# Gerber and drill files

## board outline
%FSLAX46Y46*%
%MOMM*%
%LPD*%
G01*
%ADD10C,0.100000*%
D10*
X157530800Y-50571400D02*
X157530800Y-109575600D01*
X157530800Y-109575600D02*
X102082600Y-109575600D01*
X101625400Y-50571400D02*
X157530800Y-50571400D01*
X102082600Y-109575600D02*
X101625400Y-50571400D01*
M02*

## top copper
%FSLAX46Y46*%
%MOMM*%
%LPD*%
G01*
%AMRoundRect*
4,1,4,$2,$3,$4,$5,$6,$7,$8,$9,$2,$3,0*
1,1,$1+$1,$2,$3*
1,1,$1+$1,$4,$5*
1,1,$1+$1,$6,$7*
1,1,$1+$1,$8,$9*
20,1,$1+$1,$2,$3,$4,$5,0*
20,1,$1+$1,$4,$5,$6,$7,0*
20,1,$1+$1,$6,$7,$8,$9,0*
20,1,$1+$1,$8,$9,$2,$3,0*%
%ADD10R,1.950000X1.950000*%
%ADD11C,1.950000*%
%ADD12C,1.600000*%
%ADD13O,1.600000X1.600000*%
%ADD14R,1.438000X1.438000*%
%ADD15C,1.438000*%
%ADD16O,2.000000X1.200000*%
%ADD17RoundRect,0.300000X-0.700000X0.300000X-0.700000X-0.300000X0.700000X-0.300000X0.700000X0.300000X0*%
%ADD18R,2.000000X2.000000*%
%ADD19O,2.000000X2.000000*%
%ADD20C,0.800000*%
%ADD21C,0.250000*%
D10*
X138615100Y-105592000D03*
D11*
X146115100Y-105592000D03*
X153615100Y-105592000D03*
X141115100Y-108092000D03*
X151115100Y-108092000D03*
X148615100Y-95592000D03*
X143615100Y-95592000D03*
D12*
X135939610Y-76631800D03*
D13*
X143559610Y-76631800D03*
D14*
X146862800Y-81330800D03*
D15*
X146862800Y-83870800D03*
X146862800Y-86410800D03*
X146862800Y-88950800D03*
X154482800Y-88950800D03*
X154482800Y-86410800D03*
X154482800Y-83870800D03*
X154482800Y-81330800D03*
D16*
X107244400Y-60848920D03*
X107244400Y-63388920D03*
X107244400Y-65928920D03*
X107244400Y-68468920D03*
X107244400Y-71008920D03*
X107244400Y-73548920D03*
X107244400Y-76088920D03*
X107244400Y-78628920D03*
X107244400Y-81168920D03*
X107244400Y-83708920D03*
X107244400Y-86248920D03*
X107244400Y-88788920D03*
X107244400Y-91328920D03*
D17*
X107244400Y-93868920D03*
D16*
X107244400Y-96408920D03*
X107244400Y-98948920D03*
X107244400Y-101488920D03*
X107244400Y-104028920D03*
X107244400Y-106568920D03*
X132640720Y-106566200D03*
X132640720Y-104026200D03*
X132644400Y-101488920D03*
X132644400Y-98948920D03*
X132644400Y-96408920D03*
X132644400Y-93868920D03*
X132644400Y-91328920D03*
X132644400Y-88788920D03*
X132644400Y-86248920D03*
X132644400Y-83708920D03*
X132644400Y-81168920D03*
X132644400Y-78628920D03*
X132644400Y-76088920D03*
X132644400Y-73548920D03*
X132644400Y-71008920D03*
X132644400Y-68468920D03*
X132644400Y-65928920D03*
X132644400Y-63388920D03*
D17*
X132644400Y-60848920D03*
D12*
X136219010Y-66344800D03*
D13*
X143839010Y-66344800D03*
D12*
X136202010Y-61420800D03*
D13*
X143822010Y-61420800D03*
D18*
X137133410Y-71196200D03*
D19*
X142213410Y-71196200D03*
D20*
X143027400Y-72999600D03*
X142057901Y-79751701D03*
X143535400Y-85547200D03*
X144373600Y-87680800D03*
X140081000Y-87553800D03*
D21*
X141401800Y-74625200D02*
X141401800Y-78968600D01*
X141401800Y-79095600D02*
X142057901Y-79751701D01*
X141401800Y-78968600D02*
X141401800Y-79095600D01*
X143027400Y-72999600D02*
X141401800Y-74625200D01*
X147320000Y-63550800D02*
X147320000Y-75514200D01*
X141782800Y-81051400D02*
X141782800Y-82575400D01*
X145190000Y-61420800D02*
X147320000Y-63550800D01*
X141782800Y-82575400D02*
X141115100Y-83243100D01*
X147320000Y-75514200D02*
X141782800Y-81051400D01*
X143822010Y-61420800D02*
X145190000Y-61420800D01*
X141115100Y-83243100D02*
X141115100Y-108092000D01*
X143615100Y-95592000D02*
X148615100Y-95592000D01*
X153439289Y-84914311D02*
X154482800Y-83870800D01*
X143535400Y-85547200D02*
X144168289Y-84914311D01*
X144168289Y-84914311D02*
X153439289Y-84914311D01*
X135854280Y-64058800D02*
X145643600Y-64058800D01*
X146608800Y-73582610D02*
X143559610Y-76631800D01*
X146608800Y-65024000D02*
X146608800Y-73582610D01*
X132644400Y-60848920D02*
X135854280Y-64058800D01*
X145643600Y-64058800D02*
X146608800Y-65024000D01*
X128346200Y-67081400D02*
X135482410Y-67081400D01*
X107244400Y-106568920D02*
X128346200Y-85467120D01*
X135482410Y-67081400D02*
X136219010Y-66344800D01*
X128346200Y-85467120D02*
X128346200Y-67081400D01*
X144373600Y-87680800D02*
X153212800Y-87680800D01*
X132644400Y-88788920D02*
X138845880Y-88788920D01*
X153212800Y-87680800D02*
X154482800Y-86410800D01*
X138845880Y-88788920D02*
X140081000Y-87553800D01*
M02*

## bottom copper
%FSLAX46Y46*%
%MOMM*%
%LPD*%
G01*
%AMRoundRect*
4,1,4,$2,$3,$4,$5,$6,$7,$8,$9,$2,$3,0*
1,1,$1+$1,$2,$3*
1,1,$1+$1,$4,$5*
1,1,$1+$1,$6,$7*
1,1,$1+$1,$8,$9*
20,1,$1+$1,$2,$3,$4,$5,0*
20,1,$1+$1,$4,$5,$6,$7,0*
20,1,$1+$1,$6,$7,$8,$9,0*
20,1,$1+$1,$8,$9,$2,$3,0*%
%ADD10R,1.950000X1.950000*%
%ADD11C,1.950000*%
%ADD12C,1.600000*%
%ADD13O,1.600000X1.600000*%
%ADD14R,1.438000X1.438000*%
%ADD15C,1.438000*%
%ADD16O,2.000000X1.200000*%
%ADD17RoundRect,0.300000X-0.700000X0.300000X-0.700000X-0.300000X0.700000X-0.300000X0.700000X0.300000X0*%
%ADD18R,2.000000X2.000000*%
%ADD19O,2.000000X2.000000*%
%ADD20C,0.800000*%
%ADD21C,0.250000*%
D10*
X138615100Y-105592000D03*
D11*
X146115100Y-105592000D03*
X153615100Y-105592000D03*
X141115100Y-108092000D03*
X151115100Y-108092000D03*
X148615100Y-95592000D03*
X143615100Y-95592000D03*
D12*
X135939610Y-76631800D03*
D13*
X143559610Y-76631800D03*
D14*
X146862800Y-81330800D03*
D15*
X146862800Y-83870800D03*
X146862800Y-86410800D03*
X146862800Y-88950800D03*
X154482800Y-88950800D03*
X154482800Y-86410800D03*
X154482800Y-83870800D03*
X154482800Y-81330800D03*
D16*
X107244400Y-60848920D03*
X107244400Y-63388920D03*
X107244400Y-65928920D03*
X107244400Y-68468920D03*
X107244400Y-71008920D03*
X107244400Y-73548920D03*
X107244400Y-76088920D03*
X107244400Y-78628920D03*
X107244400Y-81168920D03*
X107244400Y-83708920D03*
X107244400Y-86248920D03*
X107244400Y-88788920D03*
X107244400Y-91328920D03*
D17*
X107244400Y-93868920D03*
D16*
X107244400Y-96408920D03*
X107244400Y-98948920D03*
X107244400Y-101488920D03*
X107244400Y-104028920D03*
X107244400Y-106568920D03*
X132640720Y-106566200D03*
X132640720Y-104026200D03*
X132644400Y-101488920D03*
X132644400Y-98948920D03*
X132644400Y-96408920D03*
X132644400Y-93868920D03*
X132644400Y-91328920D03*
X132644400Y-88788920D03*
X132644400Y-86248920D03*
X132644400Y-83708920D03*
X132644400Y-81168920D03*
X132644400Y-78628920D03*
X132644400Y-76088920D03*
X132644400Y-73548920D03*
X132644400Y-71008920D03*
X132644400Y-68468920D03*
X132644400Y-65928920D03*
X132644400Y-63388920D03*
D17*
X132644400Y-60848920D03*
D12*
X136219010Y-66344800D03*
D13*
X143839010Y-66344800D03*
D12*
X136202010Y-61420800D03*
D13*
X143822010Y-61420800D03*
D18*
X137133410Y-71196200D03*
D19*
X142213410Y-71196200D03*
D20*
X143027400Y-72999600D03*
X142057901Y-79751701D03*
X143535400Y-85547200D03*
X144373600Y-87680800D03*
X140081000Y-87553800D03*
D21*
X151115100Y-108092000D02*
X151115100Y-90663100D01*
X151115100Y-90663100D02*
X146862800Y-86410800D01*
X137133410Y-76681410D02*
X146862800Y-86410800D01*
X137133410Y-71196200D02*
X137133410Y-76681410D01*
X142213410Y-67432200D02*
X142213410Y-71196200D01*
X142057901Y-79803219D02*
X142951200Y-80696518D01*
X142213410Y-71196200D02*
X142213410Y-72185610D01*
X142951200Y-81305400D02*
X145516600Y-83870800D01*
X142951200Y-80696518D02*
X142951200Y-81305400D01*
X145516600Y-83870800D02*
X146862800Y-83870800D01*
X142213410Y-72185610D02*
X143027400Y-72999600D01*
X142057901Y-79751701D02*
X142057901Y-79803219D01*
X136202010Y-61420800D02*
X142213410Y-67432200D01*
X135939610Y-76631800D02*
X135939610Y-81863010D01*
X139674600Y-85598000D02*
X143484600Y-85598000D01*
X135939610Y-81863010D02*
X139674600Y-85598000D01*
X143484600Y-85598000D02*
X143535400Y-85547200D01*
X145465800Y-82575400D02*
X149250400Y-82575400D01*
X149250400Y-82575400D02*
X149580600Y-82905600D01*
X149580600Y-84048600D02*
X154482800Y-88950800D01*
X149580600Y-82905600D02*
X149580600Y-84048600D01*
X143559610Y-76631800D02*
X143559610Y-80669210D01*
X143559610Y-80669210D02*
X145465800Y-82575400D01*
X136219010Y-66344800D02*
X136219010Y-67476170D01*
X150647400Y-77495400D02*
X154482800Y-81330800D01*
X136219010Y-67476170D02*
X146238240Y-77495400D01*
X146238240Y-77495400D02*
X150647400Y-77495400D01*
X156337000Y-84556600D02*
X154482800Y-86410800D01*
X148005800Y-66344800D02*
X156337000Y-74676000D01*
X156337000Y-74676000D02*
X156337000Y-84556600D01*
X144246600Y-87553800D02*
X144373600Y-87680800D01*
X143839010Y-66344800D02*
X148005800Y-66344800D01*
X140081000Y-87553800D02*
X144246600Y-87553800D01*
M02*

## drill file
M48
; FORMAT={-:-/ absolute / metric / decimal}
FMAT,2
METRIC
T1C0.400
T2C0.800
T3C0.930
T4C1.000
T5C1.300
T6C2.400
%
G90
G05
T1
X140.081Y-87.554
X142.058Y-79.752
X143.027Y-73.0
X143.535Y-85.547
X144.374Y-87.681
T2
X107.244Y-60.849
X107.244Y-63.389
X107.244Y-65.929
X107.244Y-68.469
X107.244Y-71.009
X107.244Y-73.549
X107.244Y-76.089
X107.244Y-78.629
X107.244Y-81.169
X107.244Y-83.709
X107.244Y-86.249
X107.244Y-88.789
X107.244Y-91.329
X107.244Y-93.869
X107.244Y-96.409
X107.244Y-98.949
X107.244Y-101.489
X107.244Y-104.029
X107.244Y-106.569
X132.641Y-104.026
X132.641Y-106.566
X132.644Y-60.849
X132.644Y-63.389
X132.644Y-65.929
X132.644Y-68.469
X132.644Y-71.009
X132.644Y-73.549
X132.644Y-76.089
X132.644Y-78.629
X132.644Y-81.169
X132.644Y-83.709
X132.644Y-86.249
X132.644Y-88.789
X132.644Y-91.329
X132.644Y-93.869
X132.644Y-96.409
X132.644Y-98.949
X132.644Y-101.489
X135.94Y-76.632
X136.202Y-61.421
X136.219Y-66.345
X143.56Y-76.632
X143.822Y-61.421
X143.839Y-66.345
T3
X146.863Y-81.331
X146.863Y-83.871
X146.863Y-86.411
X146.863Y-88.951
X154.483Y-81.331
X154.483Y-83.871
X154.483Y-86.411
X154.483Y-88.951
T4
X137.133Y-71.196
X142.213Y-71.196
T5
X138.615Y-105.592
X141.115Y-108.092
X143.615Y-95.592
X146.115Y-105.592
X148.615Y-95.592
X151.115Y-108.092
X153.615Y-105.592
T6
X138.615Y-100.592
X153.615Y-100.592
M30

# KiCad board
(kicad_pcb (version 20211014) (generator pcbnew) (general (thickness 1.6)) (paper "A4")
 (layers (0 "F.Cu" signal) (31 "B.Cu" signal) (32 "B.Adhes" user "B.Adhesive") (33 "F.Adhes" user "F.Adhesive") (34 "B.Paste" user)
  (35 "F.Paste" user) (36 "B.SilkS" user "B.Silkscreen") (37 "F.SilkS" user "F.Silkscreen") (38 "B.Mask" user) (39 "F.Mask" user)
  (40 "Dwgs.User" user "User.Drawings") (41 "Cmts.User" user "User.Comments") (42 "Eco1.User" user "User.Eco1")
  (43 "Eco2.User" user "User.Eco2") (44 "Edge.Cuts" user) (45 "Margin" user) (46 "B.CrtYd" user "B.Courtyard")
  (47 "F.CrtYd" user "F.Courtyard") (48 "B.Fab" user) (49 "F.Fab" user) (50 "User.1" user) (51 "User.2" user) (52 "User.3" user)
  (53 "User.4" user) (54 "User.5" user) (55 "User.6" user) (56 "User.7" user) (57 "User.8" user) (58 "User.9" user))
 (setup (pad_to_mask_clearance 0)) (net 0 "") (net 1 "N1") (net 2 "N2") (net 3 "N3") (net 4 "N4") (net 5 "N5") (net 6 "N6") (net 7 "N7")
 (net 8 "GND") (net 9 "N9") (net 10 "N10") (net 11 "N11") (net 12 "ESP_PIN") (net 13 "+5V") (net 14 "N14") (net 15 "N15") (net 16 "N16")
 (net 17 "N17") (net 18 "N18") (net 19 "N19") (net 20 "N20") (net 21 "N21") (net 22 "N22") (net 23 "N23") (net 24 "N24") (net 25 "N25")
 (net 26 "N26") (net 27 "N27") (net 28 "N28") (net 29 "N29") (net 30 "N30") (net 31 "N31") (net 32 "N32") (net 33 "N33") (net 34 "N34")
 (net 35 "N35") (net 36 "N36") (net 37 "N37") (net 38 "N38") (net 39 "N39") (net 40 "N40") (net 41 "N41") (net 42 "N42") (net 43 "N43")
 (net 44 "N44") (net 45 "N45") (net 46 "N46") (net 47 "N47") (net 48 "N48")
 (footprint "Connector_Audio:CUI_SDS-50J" (layer "F.Cu") (at 146.1151 100.592 180)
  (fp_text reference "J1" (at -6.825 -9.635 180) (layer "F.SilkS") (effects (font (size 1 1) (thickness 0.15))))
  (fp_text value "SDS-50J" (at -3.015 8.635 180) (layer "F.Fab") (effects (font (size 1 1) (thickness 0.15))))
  (pad "" np_thru_hole circle (at -7.5 0 180) (size 2.4 2.4) (drill 2.4) (layers *.Cu *.Mask))
  (pad "" np_thru_hole circle (at 7.5 0 180) (size 2.4 2.4) (drill 2.4) (layers *.Cu *.Mask))
  (pad "1" thru_hole rect (at 7.5 -5 180) (size 1.95 1.95) (drill 1.3) (layers *.Cu *.Mask) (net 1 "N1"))
  (pad "2" thru_hole circle (at 0 -5 180) (size 1.95 1.95) (drill 1.3) (layers *.Cu *.Mask) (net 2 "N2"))
  (pad "3" thru_hole circle (at -7.5 -5 180) (size 1.95 1.95) (drill 1.3) (layers *.Cu *.Mask) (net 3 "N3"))
  (pad "4" thru_hole circle (at 5 -7.5 180) (size 1.95 1.95) (drill 1.3) (layers *.Cu *.Mask) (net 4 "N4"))
  (pad "5" thru_hole circle (at -5 -7.5 180) (size 1.95 1.95) (drill 1.3) (layers *.Cu *.Mask) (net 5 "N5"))
  (pad "E1" thru_hole circle (at -2.5 5 180) (size 1.95 1.95) (drill 1.3) (layers *.Cu *.Mask) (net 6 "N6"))
  (pad "E2" thru_hole circle (at 2.5 5 180) (size 1.95 1.95) (drill 1.3) (layers *.Cu *.Mask) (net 6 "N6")))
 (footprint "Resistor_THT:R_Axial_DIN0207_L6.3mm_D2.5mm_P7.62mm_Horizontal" (layer "F.Cu") (at 135.93961 76.6318)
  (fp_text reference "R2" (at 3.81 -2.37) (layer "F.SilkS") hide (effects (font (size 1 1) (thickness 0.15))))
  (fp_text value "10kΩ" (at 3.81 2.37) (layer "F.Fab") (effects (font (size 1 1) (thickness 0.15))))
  (pad "1" thru_hole circle (at 0 0) (size 1.6 1.6) (drill 0.8) (layers *.Cu *.Mask) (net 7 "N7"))
  (pad "2" thru_hole oval (at 7.62 0) (size 1.6 1.6) (drill 0.8) (layers *.Cu *.Mask) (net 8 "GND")))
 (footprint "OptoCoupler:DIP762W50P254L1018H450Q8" (layer "F.Cu") (at 150.6728 85.1408)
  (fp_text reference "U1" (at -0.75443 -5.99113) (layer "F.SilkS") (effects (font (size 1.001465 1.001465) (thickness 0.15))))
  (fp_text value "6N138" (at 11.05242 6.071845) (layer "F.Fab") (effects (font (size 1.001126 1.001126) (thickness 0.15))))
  (pad "1" thru_hole rect locked (at -3.81 -3.81) (size 1.438 1.438) (drill 0.93) (layers *.Cu *.Mask) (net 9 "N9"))
  (pad "2" thru_hole circle locked (at -3.81 -1.27) (size 1.438 1.438) (drill 0.93) (layers *.Cu *.Mask) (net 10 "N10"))
  (pad "3" thru_hole circle locked (at -3.81 1.27) (size 1.438 1.438) (drill 0.93) (layers *.Cu *.Mask) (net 5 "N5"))
  (pad "4" thru_hole circle locked (at -3.81 3.81) (size 1.438 1.438) (drill 0.93) (layers *.Cu *.Mask) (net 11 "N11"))
  (pad "5" thru_hole circle locked (at 3.81 3.81) (size 1.438 1.438) (drill 0.93) (layers *.Cu *.Mask) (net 8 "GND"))
  (pad "6" thru_hole circle locked (at 3.81 1.27) (size 1.438 1.438) (drill 0.93) (layers *.Cu *.Mask) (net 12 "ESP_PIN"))
  (pad "7" thru_hole circle locked (at 3.81 -1.27) (size 1.438 1.438) (drill 0.93) (layers *.Cu *.Mask) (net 7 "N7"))
  (pad "8" thru_hole circle locked (at 3.81 -3.81) (size 1.438 1.438) (drill 0.93) (layers *.Cu *.Mask) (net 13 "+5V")))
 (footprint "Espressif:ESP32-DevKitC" (layer "F.Cu") (at 107.24072 60.8462)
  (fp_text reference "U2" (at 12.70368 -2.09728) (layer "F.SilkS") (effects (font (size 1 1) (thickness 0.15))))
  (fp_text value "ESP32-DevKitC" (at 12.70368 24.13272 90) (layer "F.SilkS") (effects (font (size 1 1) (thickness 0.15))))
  (pad "1" thru_hole oval (at 0.00368 0.00272 270) (size 1.2 2) (drill 0.8) (layers *.Cu *.Mask) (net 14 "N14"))
  (pad "2" thru_hole oval (at 0.00368 2.54272 270) (size 1.2 2) (drill 0.8) (layers *.Cu *.Mask) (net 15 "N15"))
  (pad "3" thru_hole oval (at 0.00368 5.08272 270) (size 1.2 2) (drill 0.8) (layers *.Cu *.Mask) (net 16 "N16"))
  (pad "4" thru_hole oval (at 0.00368 7.62272 270) (size 1.2 2) (drill 0.8) (layers *.Cu *.Mask) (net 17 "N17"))
  (pad "5" thru_hole oval (at 0.00368 10.16272 270) (size 1.2 2) (drill 0.8) (layers *.Cu *.Mask) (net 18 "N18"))
  (pad "6" thru_hole oval (at 0.00368 12.70272 270) (size 1.2 2) (drill 0.8) (layers *.Cu *.Mask) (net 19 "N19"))
  (pad "7" thru_hole oval (at 0.00368 15.24272 270) (size 1.2 2) (drill 0.8) (layers *.Cu *.Mask) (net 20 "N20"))
  (pad "8" thru_hole oval (at 0.00368 17.78272 270) (size 1.2 2) (drill 0.8) (layers *.Cu *.Mask) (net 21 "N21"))
  (pad "9" thru_hole oval (at 0.00368 20.32272 270) (size 1.2 2) (drill 0.8) (layers *.Cu *.Mask) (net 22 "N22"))
  (pad "10" thru_hole oval (at 0.00368 22.86272 270) (size 1.2 2) (drill 0.8) (layers *.Cu *.Mask) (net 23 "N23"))
  (pad "11" thru_hole oval (at 0.00368 25.40272 270) (size 1.2 2) (drill 0.8) (layers *.Cu *.Mask) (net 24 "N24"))
  (pad "12" thru_hole oval (at 0.00368 27.94272 270) (size 1.2 2) (drill 0.8) (layers *.Cu *.Mask) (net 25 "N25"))
  (pad "13" thru_hole oval (at 0.00368 30.48272 270) (size 1.2 2) (drill 0.8) (layers *.Cu *.Mask) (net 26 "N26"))
  (pad "14" thru_hole roundrect (at 0.00368 33.02272 270) (size 1.2 2) (drill 0.8) (layers *.Cu *.Mask) (roundrect_rratio 0.25)
   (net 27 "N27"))
  (pad "15" thru_hole oval (at 0.00368 35.56272 270) (size 1.2 2) (drill 0.8) (layers *.Cu *.Mask) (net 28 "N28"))
  (pad "16" thru_hole oval (at 0.00368 38.10272 270) (size 1.2 2) (drill 0.8) (layers *.Cu *.Mask) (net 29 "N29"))
  (pad "17" thru_hole oval (at 0.00368 40.64272 270) (size 1.2 2) (drill 0.8) (layers *.Cu *.Mask) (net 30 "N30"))
  (pad "18" thru_hole oval (at 0.00368 43.18272 270) (size 1.2 2) (drill 0.8) (layers *.Cu *.Mask) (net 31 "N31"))
  (pad "19" thru_hole oval (at 0.00368 45.72272 270) (size 1.2 2) (drill 0.8) (layers *.Cu *.Mask) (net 13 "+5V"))
  (pad "20" thru_hole oval (at 25.4 45.72 270) (size 1.2 2) (drill 0.8) (layers *.Cu *.Mask) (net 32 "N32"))
  (pad "21" thru_hole oval (at 25.4 43.18 270) (size 1.2 2) (drill 0.8) (layers *.Cu *.Mask) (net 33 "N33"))
  (pad "22" thru_hole oval (at 25.40368 40.64272 270) (size 1.2 2) (drill 0.8) (layers *.Cu *.Mask) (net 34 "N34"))
  (pad "23" thru_hole oval (at 25.40368 38.10272 270) (size 1.2 2) (drill 0.8) (layers *.Cu *.Mask) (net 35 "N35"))
  (pad "24" thru_hole oval (at 25.40368 35.56272 270) (size 1.2 2) (drill 0.8) (layers *.Cu *.Mask) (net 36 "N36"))
  (pad "25" thru_hole oval (at 25.40368 33.02272 270) (size 1.2 2) (drill 0.8) (layers *.Cu *.Mask) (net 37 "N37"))
  (pad "26" thru_hole oval (at 25.40368 30.48272 270) (size 1.2 2) (drill 0.8) (layers *.Cu *.Mask) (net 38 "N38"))
  (pad "27" thru_hole oval (at 25.40368 27.94272 270) (size 1.2 2) (drill 0.8) (layers *.Cu *.Mask) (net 12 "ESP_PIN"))
  (pad "28" thru_hole oval (at 25.40368 25.40272 270) (size 1.2 2) (drill 0.8) (layers *.Cu *.Mask) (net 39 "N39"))
  (pad "29" thru_hole oval (at 25.40368 22.86272 270) (size 1.2 2) (drill 0.8) (layers *.Cu *.Mask) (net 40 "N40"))
  (pad "30" thru_hole oval (at 25.40368 20.32272 270) (size 1.2 2) (drill 0.8) (layers *.Cu *.Mask) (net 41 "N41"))
  (pad "31" thru_hole oval (at 25.40368 17.78272 270) (size 1.2 2) (drill 0.8) (layers *.Cu *.Mask) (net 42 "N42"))
  (pad "32" thru_hole oval (at 25.40368 15.24272 270) (size 1.2 2) (drill 0.8) (layers *.Cu *.Mask) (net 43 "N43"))
  (pad "33" thru_hole oval (at 25.40368 12.70272 270) (size 1.2 2) (drill 0.8) (layers *.Cu *.Mask) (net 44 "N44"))
  (pad "34" thru_hole oval (at 25.40368 10.16272 270) (size 1.2 2) (drill 0.8) (layers *.Cu *.Mask) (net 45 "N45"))
  (pad "35" thru_hole oval (at 25.40368 7.62272 270) (size 1.2 2) (drill 0.8) (layers *.Cu *.Mask) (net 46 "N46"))
  (pad "36" thru_hole oval (at 25.40368 5.08272 270) (size 1.2 2) (drill 0.8) (layers *.Cu *.Mask) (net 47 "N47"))
  (pad "37" thru_hole oval (at 25.40368 2.54272 270) (size 1.2 2) (drill 0.8) (layers *.Cu *.Mask) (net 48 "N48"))
  (pad "38" thru_hole roundrect (at 25.40368 0.00272 270) (size 1.2 2) (drill 0.8) (layers *.Cu *.Mask) (roundrect_rratio 0.25)
   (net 8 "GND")))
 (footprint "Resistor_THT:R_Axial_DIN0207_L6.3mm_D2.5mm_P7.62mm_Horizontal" (layer "F.Cu") (at 136.21901 66.3448)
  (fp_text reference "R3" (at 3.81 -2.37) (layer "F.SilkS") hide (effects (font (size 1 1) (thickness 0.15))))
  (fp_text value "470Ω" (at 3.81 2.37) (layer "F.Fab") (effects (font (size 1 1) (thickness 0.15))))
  (pad "1" thru_hole circle (at 0 0) (size 1.6 1.6) (drill 0.8) (layers *.Cu *.Mask) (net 13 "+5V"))
  (pad "2" thru_hole oval (at 7.62 0) (size 1.6 1.6) (drill 0.8) (layers *.Cu *.Mask) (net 12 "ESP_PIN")))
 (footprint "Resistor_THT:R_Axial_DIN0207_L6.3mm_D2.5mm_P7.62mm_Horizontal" (layer "F.Cu") (at 136.20201 61.4208)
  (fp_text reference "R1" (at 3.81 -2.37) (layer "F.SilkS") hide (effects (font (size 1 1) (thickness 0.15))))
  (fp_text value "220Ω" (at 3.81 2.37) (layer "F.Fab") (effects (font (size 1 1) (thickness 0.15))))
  (pad "1" thru_hole circle (at 0 0) (size 1.6 1.6) (drill 0.8) (layers *.Cu *.Mask) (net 10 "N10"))
  (pad "2" thru_hole oval (at 7.62 0) (size 1.6 1.6) (drill 0.8) (layers *.Cu *.Mask) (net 4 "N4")))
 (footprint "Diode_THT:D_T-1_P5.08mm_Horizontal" (layer "F.Cu") (at 137.13341 71.1962)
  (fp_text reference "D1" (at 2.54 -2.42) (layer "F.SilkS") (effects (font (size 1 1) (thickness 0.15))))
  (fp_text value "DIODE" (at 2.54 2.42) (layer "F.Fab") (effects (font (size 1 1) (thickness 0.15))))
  (pad "1" thru_hole rect (at 0 0) (size 2 2) (drill 1) (layers *.Cu *.Mask) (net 5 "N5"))
  (pad "2" thru_hole oval (at 5.08 0) (size 2 2) (drill 1) (layers *.Cu *.Mask) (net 10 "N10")))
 (gr_line (start 157.5308 50.5714) (end 157.5308 109.5756) (layer "Edge.Cuts") (width 0.1))
 (gr_line (start 157.5308 109.5756) (end 102.0826 109.5756) (layer "Edge.Cuts") (width 0.1))
 (gr_line (start 101.6254 50.5714) (end 157.5308 50.5714) (layer "Edge.Cuts") (width 0.1))
 (gr_line (start 102.0826 109.5756) (end 101.6254 50.5714) (layer "Edge.Cuts") (width 0.1))
 (segment (start 151.1151 108.092) (end 151.1151 90.6631) (width 0.25) (layer "B.Cu") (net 5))
 (segment (start 151.1151 90.6631) (end 146.8628 86.4108) (width 0.25) (layer "B.Cu") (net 5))
 (segment (start 137.13341 76.68141) (end 146.8628 86.4108) (width 0.25) (layer "B.Cu") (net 5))
 (segment (start 137.13341 71.1962) (end 137.13341 76.68141) (width 0.25) (layer "B.Cu") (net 5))
 (segment (start 141.4018 74.6252) (end 141.4018 78.9686) (width 0.25) (layer "F.Cu") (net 10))
 (segment (start 141.4018 79.0956) (end 142.057901 79.751701) (width 0.25) (layer "F.Cu") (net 10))
 (segment (start 141.4018 78.9686) (end 141.4018 79.0956) (width 0.25) (layer "F.Cu") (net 10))
 (segment (start 143.0274 72.9996) (end 141.4018 74.6252) (width 0.25) (layer "F.Cu") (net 10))
 (via (at 143.0274 72.9996) (size 0.8) (drill 0.4) (layers "F.Cu" "B.Cu") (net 10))
 (via (at 142.057901 79.751701) (size 0.8) (drill 0.4) (layers "F.Cu" "B.Cu") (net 10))
 (segment (start 142.21341 67.4322) (end 142.21341 71.1962) (width 0.25) (layer "B.Cu") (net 10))
 (segment (start 142.057901 79.803219) (end 142.9512 80.696518) (width 0.25) (layer "B.Cu") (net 10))
 (segment (start 142.21341 71.1962) (end 142.21341 72.18561) (width 0.25) (layer "B.Cu") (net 10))
 (segment (start 142.9512 81.3054) (end 145.5166 83.8708) (width 0.25) (layer "B.Cu") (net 10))
 (segment (start 142.9512 80.696518) (end 142.9512 81.3054) (width 0.25) (layer "B.Cu") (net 10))
 (segment (start 145.5166 83.8708) (end 146.8628 83.8708) (width 0.25) (layer "B.Cu") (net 10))
 (segment (start 142.21341 72.18561) (end 143.0274 72.9996) (width 0.25) (layer "B.Cu") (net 10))
 (segment (start 142.057901 79.751701) (end 142.057901 79.803219) (width 0.25) (layer "B.Cu") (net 10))
 (segment (start 136.20201 61.4208) (end 142.21341 67.4322) (width 0.25) (layer "B.Cu") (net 10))
 (segment (start 147.32 63.5508) (end 147.32 75.5142) (width 0.25) (layer "F.Cu") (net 4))
 (segment (start 141.7828 81.0514) (end 141.7828 82.5754) (width 0.25) (layer "F.Cu") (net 4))
 (segment (start 145.19 61.4208) (end 147.32 63.5508) (width 0.25) (layer "F.Cu") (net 4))
 (segment (start 141.7828 82.5754) (end 141.1151 83.2431) (width 0.25) (layer "F.Cu") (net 4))
 (segment (start 147.32 75.5142) (end 141.7828 81.0514) (width 0.25) (layer "F.Cu") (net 4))
 (segment (start 143.82201 61.4208) (end 145.19 61.4208) (width 0.25) (layer "F.Cu") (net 4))
 (segment (start 141.1151 83.2431) (end 141.1151 108.092) (width 0.25) (layer "F.Cu") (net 4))
 (segment (start 143.6151 95.592) (end 148.6151 95.592) (width 0.25) (layer "F.Cu") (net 6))
 (segment (start 153.439289 84.914311) (end 154.4828 83.8708) (width 0.25) (layer "F.Cu") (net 7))
 (segment (start 143.5354 85.5472) (end 144.168289 84.914311) (width 0.25) (layer "F.Cu") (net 7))
 (segment (start 144.168289 84.914311) (end 153.439289 84.914311) (width 0.25) (layer "F.Cu") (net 7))
 (via (at 143.5354 85.5472) (size 0.8) (drill 0.4) (layers "F.Cu" "B.Cu") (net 7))
 (segment (start 135.93961 76.6318) (end 135.93961 81.86301) (width 0.25) (layer "B.Cu") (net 7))
 (segment (start 139.6746 85.598) (end 143.4846 85.598) (width 0.25) (layer "B.Cu") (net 7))
 (segment (start 135.93961 81.86301) (end 139.6746 85.598) (width 0.25) (layer "B.Cu") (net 7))
 (segment (start 143.4846 85.598) (end 143.5354 85.5472) (width 0.25) (layer "B.Cu") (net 7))
 (segment (start 135.85428 64.0588) (end 145.6436 64.0588) (width 0.25) (layer "F.Cu") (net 8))
 (segment (start 146.6088 73.58261) (end 143.55961 76.6318) (width 0.25) (layer "F.Cu") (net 8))
 (segment (start 146.6088 65.024) (end 146.6088 73.58261) (width 0.25) (layer "F.Cu") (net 8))
 (segment (start 132.6444 60.84892) (end 135.85428 64.0588) (width 0.25) (layer "F.Cu") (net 8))
 (segment (start 145.6436 64.0588) (end 146.6088 65.024) (width 0.25) (layer "F.Cu") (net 8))
 (segment (start 145.4658 82.5754) (end 149.2504 82.5754) (width 0.25) (layer "B.Cu") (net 8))
 (segment (start 149.2504 82.5754) (end 149.5806 82.9056) (width 0.25) (layer "B.Cu") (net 8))
 (segment (start 149.5806 84.0486) (end 154.4828 88.9508) (width 0.25) (layer "B.Cu") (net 8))
 (segment (start 149.5806 82.9056) (end 149.5806 84.0486) (width 0.25) (layer "B.Cu") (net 8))
 (segment (start 143.55961 76.6318) (end 143.55961 80.66921) (width 0.25) (layer "B.Cu") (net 8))
 (segment (start 143.55961 80.66921) (end 145.4658 82.5754) (width 0.25) (layer "B.Cu") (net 8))
 (segment (start 128.3462 67.0814) (end 135.48241 67.0814) (width 0.25) (layer "F.Cu") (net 13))
 (segment (start 107.2444 106.56892) (end 128.3462 85.46712) (width 0.25) (layer "F.Cu") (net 13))
 (segment (start 135.48241 67.0814) (end 136.21901 66.3448) (width 0.25) (layer "F.Cu") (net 13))
 (segment (start 128.3462 85.46712) (end 128.3462 67.0814) (width 0.25) (layer "F.Cu") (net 13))
 (segment (start 136.21901 66.3448) (end 136.21901 67.47617) (width 0.25) (layer "B.Cu") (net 13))
 (segment (start 150.6474 77.4954) (end 154.4828 81.3308) (width 0.25) (layer "B.Cu") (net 13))
 (segment (start 136.21901 67.47617) (end 146.23824 77.4954) (width 0.25) (layer "B.Cu") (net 13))
 (segment (start 146.23824 77.4954) (end 150.6474 77.4954) (width 0.25) (layer "B.Cu") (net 13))
 (segment (start 144.3736 87.6808) (end 153.2128 87.6808) (width 0.25) (layer "F.Cu") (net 12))
 (segment (start 132.6444 88.78892) (end 138.84588 88.78892) (width 0.25) (layer "F.Cu") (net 12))
 (segment (start 153.2128 87.6808) (end 154.4828 86.4108) (width 0.25) (layer "F.Cu") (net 12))
 (segment (start 138.84588 88.78892) (end 140.081 87.5538) (width 0.25) (layer "F.Cu") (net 12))
 (via (at 144.3736 87.6808) (size 0.8) (drill 0.4) (layers "F.Cu" "B.Cu") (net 12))
 (via (at 140.081 87.5538) (size 0.8) (drill 0.4) (layers "F.Cu" "B.Cu") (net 12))
 (segment (start 156.337 84.5566) (end 154.4828 86.4108) (width 0.25) (layer "B.Cu") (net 12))
 (segment (start 148.0058 66.3448) (end 156.337 74.676) (width 0.25) (layer "B.Cu") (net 12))
 (segment (start 156.337 74.676) (end 156.337 84.5566) (width 0.25) (layer "B.Cu") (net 12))
 (segment (start 144.2466 87.5538) (end 144.3736 87.6808) (width 0.25) (layer "B.Cu") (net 12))
 (segment (start 143.83901 66.3448) (end 148.0058 66.3448) (width 0.25) (layer "B.Cu") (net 12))
 (segment (start 140.081 87.5538) (end 144.2466 87.5538) (width 0.25) (layer "B.Cu") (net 12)))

